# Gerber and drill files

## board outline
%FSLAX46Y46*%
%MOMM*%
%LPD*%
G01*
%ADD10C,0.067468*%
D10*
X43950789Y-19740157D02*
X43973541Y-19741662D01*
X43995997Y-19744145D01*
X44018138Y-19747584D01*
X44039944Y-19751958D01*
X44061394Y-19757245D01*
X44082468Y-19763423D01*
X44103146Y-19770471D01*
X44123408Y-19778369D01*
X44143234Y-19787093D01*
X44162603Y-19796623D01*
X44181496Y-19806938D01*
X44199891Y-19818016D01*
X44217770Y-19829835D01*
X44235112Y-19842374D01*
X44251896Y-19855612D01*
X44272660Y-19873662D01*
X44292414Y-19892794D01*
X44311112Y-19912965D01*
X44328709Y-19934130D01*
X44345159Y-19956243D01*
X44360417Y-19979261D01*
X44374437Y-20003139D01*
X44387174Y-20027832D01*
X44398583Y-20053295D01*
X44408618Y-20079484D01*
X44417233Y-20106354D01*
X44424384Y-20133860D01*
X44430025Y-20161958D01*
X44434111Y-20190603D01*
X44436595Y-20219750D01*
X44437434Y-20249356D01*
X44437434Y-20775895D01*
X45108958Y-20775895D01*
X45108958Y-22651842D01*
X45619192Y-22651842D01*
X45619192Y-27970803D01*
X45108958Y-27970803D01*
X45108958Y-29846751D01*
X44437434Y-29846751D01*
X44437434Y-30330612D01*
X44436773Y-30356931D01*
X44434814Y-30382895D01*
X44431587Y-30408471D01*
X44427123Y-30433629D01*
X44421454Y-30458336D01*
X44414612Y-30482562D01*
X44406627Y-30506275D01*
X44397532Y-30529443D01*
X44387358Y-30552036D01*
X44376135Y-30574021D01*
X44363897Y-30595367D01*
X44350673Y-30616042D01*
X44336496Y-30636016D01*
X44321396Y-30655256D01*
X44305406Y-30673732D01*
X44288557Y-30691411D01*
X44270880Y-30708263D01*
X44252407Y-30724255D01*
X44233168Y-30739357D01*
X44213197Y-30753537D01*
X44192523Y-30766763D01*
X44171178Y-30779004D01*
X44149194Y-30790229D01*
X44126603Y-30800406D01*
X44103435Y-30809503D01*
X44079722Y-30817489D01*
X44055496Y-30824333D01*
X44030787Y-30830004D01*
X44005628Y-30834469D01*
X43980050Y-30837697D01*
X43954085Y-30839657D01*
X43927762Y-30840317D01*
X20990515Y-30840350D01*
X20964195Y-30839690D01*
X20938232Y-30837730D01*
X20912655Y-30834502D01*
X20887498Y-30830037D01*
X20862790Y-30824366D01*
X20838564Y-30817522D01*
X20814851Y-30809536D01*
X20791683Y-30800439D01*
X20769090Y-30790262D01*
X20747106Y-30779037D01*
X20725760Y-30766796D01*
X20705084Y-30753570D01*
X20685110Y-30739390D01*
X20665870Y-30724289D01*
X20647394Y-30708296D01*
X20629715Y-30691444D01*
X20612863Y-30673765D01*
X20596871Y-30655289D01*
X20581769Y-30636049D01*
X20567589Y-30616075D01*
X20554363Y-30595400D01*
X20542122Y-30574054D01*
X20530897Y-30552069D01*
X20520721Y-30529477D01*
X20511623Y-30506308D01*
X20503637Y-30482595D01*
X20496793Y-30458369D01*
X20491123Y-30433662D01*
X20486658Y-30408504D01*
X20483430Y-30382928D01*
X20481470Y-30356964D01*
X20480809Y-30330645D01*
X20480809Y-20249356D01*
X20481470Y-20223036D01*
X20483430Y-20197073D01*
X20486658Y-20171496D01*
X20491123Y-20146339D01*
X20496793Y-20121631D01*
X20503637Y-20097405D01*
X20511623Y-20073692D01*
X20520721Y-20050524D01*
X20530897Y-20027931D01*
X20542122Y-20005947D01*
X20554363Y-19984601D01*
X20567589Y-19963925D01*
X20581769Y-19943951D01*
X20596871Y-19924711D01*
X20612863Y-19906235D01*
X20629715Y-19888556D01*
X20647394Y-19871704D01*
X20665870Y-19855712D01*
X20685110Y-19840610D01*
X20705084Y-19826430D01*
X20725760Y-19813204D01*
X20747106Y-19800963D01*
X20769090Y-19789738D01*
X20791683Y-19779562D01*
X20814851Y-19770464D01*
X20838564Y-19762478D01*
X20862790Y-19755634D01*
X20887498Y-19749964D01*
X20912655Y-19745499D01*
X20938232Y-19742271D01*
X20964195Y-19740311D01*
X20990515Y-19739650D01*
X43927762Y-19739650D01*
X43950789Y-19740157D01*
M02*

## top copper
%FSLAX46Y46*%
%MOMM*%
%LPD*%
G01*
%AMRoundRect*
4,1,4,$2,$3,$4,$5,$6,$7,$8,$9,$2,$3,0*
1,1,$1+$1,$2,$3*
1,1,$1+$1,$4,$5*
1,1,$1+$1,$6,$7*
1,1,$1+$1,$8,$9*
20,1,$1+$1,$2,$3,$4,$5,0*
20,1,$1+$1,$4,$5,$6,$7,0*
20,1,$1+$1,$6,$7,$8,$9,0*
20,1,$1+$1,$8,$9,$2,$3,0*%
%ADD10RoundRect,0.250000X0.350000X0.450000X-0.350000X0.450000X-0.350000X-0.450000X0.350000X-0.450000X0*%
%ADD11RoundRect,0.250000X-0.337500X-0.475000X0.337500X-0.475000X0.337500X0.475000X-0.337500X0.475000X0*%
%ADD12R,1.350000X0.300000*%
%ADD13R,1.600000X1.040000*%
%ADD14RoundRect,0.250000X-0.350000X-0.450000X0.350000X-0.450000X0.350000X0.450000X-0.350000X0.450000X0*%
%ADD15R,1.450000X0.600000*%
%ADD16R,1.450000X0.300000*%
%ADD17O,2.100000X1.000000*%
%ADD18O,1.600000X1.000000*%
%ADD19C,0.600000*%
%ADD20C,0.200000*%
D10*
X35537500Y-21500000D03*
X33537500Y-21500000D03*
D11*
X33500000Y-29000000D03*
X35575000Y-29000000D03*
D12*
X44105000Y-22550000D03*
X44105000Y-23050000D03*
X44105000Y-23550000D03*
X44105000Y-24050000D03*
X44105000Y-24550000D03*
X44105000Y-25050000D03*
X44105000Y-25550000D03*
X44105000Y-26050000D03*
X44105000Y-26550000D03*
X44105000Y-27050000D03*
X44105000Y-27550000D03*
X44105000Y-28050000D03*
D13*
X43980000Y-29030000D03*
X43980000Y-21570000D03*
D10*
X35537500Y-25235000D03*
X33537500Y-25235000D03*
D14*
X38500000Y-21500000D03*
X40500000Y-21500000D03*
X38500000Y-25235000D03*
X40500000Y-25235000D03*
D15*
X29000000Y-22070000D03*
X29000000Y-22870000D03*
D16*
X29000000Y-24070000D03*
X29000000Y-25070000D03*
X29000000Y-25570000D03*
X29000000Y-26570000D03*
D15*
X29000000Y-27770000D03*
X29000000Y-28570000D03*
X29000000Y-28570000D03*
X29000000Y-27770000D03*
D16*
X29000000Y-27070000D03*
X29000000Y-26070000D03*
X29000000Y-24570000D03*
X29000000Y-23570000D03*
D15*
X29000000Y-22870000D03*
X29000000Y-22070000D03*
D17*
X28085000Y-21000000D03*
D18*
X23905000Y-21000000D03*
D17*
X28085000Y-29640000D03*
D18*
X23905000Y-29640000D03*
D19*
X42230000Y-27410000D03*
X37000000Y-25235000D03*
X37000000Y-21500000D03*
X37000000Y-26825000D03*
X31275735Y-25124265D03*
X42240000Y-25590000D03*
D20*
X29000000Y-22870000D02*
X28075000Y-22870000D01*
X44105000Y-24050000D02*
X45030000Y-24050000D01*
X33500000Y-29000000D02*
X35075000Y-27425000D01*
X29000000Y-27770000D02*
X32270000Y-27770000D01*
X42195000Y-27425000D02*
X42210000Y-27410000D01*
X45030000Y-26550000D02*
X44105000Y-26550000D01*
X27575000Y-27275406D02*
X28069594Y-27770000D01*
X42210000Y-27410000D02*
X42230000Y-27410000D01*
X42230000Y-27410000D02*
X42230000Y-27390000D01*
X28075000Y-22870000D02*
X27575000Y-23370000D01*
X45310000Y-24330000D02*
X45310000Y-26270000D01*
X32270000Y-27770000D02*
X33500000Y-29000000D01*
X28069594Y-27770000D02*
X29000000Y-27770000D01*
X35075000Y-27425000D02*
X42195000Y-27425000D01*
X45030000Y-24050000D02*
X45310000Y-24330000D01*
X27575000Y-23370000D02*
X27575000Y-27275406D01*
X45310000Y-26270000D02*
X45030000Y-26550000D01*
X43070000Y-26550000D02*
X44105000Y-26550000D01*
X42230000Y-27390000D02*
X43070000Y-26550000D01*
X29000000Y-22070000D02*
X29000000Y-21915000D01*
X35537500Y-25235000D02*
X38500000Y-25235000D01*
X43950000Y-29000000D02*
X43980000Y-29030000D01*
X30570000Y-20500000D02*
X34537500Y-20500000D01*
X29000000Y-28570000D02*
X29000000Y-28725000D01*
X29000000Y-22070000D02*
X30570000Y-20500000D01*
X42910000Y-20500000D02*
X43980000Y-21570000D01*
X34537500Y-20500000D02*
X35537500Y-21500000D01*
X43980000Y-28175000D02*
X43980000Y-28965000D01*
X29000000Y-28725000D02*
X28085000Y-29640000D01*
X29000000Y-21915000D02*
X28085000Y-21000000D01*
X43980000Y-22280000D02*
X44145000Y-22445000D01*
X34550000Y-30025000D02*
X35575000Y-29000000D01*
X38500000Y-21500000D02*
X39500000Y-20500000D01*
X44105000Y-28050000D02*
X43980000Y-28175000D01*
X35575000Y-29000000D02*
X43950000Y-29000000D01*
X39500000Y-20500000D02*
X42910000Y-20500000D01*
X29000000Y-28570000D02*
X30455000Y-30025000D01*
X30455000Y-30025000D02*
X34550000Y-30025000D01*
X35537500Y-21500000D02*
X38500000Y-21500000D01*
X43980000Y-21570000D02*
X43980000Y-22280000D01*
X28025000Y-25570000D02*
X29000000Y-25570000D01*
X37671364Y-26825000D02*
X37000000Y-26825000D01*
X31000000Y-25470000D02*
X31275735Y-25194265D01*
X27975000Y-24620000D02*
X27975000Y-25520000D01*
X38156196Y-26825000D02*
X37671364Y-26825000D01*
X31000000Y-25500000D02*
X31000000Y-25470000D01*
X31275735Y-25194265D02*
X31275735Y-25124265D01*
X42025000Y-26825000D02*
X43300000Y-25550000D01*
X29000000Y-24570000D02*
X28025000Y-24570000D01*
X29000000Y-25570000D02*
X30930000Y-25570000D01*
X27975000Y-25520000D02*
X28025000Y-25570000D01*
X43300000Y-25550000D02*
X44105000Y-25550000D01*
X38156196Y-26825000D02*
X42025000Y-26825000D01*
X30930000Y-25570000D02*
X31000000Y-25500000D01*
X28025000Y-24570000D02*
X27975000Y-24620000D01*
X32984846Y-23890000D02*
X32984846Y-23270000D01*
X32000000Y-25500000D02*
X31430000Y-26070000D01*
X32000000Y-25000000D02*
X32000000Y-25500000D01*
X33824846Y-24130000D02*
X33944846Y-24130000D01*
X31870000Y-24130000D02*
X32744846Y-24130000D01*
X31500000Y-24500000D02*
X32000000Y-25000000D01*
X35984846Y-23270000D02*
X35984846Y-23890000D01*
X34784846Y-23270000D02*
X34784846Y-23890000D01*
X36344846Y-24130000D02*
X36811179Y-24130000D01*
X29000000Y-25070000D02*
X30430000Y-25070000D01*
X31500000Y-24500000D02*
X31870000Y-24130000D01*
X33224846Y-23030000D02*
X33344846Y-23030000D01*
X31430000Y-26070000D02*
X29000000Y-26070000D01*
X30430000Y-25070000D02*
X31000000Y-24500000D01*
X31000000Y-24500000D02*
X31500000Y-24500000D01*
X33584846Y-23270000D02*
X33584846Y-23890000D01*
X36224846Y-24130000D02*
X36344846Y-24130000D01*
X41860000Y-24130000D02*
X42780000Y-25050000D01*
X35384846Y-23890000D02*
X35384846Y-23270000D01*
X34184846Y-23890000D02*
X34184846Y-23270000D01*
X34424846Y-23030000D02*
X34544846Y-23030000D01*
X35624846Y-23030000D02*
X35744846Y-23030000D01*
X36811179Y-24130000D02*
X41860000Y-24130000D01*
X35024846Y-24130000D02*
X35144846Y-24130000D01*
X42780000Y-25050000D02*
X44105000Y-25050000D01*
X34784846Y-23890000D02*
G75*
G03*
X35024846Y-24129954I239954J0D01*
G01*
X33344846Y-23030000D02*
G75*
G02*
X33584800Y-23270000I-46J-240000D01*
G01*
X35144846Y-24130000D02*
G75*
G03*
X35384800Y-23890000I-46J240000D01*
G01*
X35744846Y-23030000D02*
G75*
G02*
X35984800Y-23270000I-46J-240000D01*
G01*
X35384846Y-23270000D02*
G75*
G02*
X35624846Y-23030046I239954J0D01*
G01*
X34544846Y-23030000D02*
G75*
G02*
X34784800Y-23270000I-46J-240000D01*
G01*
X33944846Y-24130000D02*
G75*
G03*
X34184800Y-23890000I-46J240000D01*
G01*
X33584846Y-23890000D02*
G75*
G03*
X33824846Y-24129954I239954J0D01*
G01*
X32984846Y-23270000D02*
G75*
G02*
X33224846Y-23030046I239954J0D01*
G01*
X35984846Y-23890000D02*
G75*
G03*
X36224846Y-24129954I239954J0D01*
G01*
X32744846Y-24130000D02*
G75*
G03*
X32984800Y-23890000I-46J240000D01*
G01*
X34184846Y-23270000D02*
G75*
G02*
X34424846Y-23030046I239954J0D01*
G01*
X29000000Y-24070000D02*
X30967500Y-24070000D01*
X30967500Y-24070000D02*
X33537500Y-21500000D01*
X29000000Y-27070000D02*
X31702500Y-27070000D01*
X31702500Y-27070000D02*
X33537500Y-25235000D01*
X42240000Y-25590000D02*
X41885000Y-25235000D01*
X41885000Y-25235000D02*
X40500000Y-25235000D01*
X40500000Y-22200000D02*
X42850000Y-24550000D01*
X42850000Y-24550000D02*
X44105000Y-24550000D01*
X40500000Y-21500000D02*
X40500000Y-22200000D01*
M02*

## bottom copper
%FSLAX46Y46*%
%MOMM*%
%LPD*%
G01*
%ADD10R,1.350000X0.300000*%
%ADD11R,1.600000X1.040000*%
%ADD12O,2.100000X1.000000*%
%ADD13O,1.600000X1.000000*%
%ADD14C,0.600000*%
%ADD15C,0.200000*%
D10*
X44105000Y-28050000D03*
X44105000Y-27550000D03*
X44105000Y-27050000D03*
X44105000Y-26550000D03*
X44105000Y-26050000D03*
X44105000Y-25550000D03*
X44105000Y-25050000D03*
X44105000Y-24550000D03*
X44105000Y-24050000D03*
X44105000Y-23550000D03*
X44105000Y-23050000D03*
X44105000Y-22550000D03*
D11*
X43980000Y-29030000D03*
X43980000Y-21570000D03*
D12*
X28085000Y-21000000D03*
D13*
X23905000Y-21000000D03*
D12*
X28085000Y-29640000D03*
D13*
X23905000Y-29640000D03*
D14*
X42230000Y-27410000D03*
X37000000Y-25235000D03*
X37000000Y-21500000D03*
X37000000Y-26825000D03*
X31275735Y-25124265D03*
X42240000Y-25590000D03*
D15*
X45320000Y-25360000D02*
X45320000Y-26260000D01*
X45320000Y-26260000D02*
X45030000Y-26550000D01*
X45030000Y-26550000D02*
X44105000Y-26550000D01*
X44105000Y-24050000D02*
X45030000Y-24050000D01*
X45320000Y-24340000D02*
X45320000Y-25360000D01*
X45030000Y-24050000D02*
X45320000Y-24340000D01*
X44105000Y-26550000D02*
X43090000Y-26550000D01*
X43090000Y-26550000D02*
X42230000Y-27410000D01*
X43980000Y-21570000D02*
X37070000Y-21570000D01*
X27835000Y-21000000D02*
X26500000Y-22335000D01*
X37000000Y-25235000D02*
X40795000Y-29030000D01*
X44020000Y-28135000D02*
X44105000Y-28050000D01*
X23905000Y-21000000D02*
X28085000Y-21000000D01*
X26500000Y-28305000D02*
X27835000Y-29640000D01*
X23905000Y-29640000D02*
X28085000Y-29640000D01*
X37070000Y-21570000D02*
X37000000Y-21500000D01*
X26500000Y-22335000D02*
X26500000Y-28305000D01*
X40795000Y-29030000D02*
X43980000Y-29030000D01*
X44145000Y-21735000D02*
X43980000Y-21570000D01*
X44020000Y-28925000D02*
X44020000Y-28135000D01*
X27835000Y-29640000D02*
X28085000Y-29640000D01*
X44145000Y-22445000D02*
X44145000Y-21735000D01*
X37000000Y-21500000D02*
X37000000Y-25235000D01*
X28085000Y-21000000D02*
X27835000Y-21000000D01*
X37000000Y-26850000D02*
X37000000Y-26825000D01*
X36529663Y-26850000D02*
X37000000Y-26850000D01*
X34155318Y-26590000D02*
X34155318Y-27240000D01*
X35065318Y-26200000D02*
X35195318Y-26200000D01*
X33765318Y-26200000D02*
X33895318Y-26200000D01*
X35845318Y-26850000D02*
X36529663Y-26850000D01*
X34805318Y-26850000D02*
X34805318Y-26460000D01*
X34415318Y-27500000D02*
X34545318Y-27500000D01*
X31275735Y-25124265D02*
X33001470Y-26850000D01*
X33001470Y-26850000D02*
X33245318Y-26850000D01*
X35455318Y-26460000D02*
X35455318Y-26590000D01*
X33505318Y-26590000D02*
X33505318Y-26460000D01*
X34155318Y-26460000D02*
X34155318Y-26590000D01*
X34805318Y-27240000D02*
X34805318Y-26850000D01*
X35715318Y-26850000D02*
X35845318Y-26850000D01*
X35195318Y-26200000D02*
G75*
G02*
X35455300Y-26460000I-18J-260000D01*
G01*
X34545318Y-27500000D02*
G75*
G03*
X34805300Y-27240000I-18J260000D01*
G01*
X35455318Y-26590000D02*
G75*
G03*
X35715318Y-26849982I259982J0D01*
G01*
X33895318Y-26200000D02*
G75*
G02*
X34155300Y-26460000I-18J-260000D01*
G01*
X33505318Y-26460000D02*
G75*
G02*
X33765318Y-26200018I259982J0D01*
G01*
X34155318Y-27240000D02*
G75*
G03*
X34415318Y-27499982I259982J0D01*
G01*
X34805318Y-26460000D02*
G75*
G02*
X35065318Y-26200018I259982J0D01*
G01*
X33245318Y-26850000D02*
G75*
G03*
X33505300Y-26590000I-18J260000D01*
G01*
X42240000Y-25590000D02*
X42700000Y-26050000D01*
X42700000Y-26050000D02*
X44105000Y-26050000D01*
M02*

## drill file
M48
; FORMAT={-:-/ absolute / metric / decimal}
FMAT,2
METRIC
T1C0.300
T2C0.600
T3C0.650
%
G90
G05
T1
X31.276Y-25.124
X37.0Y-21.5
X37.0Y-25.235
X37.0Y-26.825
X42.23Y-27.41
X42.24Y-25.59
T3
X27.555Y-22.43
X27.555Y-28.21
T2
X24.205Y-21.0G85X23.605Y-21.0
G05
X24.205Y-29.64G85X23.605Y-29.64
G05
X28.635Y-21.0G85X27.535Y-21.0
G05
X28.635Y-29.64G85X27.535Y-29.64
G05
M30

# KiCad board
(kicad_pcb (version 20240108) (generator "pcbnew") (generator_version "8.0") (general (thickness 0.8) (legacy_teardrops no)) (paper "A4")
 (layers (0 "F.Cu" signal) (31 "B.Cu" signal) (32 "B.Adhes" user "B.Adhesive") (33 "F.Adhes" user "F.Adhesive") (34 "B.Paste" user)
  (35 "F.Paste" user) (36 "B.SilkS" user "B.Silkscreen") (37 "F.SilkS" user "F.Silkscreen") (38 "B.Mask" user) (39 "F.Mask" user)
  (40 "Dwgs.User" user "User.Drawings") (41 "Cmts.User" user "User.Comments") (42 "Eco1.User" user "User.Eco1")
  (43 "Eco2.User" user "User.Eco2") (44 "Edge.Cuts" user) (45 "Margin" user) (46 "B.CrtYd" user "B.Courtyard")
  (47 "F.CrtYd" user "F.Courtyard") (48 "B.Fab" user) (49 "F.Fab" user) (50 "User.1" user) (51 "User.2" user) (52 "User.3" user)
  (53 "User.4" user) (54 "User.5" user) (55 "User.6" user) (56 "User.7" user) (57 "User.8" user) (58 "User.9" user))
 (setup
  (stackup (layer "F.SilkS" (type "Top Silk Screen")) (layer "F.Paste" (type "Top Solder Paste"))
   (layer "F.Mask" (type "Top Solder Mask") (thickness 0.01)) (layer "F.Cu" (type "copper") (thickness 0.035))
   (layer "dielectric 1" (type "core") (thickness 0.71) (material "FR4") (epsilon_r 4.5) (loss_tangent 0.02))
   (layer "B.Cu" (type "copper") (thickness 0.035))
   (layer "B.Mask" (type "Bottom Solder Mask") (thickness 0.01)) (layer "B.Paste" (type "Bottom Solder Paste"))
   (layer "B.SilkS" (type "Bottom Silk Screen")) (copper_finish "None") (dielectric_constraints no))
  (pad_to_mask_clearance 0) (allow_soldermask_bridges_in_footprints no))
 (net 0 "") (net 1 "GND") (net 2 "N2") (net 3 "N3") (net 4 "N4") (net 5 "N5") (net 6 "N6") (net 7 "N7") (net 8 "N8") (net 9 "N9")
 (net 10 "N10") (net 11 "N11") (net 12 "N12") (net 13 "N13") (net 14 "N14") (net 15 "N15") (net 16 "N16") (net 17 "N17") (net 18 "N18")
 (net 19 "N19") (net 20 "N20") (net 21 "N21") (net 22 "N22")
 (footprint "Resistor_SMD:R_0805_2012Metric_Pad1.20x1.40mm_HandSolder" (layer "F.Cu") (at 34.5375 21.5 180)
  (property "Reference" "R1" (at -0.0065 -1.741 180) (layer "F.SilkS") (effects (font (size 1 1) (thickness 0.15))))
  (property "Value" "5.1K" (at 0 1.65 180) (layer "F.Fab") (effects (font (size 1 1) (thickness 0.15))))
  (pad "1" smd roundrect (at -1 0 180) (size 1.2 1.4) (layers "F.Cu" "F.Paste" "F.Mask") (roundrect_rratio 0.208333) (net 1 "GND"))
  (pad "2" smd roundrect (at 1 0 180) (size 1.2 1.4) (layers "F.Cu" "F.Paste" "F.Mask") (roundrect_rratio 0.208333) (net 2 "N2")))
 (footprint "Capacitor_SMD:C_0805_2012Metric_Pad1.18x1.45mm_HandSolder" (layer "F.Cu") (at 34.5375 29)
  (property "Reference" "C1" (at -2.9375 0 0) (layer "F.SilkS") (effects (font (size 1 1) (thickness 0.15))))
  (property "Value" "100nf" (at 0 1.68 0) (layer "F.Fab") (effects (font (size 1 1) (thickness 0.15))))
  (pad "1" smd roundrect (at -1.0375 0) (size 1.175 1.45) (layers "F.Cu" "F.Paste" "F.Mask") (roundrect_rratio 0.212766) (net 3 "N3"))
  (pad "2" smd roundrect (at 1.0375 0) (size 1.175 1.45) (layers "F.Cu" "F.Paste" "F.Mask") (roundrect_rratio 0.212766) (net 1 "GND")))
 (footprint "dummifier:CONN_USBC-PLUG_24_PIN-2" (layer "F.Cu") (at 44.95 25.33 90)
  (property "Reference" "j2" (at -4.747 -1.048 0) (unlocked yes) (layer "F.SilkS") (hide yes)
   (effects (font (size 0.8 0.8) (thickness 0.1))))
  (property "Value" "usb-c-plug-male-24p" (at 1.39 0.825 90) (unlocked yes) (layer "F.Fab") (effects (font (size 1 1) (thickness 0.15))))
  (pad "A1" smd rect (at 2.78 -0.845 90) (size 0.3 1.35) (layers "F.Cu" "F.Paste" "F.Mask") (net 1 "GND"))
  (pad "A2" smd rect (at 2.28 -0.845 90) (size 0.3 1.35) (layers "F.Cu" "F.Paste" "F.Mask") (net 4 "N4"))
  (pad "A3" smd rect (at 1.78 -0.845 90) (size 0.3 1.35) (layers "F.Cu" "F.Paste" "F.Mask") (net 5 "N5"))
  (pad "A4" smd rect (at 1.28 -0.845 90) (size 0.3 1.35) (layers "F.Cu" "F.Paste" "F.Mask") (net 3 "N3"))
  (pad "A5" smd rect (at 0.78 -0.845 90) (size 0.3 1.35) (layers "F.Cu" "F.Paste" "F.Mask") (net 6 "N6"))
  (pad "A6" smd rect (at 0.28 -0.845 90) (size 0.3 1.35) (layers "F.Cu" "F.Paste" "F.Mask") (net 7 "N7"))
  (pad "A7" smd rect (at -0.22 -0.845 90) (size 0.3 1.35) (layers "F.Cu" "F.Paste" "F.Mask") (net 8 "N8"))
  (pad "A8" smd rect (at -0.72 -0.845 90) (size 0.3 1.35) (layers "F.Cu" "F.Paste" "F.Mask") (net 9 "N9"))
  (pad "A9" smd rect (at -1.22 -0.845 90) (size 0.3 1.35) (layers "F.Cu" "F.Paste" "F.Mask") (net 3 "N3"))
  (pad "A10" smd rect (at -1.72 -0.845 90) (size 0.3 1.35) (layers "F.Cu" "F.Paste" "F.Mask") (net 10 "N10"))
  (pad "A11" smd rect (at -2.22 -0.845 90) (size 0.3 1.35) (layers "F.Cu" "F.Paste" "F.Mask") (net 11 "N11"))
  (pad "A12" smd rect (at -2.72 -0.845 90) (size 0.3 1.35) (layers "F.Cu" "F.Paste" "F.Mask") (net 1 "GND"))
  (pad "B1" smd rect (at -2.72 -0.845 90) (size 0.3 1.35) (layers "B.Cu" "B.Paste" "B.Mask") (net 1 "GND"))
  (pad "B2" smd rect (at -2.22 -0.845 90) (size 0.3 1.35) (layers "B.Cu" "B.Paste" "B.Mask") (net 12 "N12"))
  (pad "B3" smd rect (at -1.72 -0.845 90) (size 0.3 1.35) (layers "B.Cu" "B.Paste" "B.Mask") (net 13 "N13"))
  (pad "B4" smd rect (at -1.22 -0.845 90) (size 0.3 1.35) (layers "B.Cu" "B.Paste" "B.Mask") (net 3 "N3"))
  (pad "B5" smd rect (at -0.72 -0.845 90) (size 0.3 1.35) (layers "B.Cu" "B.Paste" "B.Mask") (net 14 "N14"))
  (pad "B6" smd rect (at -0.22 -0.845 90) (size 0.3 1.35) (layers "B.Cu" "B.Paste" "B.Mask") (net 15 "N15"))
  (pad "B7" smd rect (at 0.28 -0.845 90) (size 0.3 1.35) (layers "B.Cu" "B.Paste" "B.Mask") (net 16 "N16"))
  (pad "B8" smd rect (at 0.78 -0.845 90) (size 0.3 1.35) (layers "B.Cu" "B.Paste" "B.Mask") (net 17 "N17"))
  (pad "B9" smd rect (at 1.28 -0.845 90) (size 0.3 1.35) (layers "B.Cu" "B.Paste" "B.Mask") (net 3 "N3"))
  (pad "B10" smd rect (at 1.78 -0.845 90) (size 0.3 1.35) (layers "B.Cu" "B.Paste" "B.Mask") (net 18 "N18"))
  (pad "B11" smd rect (at 2.28 -0.845 90) (size 0.3 1.35) (layers "B.Cu" "B.Paste" "B.Mask") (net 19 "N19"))
  (pad "B12" smd rect (at 2.78 -0.845 90) (size 0.3 1.35) (layers "B.Cu" "B.Paste" "B.Mask") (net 1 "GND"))
  (pad "S" smd rect (at -3.7 -0.97 90) (size 1.04 1.6) (layers "F.Cu" "F.Paste" "F.Mask") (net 1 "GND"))
  (pad "S" smd rect (at -3.7 -0.97 90) (size 1.04 1.6) (layers "B.Cu" "B.Paste" "B.Mask") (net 1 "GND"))
  (pad "S" smd rect (at 3.76 -0.97 90) (size 1.04 1.6) (layers "F.Cu" "F.Paste" "F.Mask") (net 1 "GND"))
  (pad "S" smd rect (at 3.76 -0.97 90) (size 1.04 1.6) (layers "B.Cu" "B.Paste" "B.Mask") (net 1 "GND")))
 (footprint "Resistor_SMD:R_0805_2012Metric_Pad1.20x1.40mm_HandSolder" (layer "F.Cu") (at 34.5375 25.235 180)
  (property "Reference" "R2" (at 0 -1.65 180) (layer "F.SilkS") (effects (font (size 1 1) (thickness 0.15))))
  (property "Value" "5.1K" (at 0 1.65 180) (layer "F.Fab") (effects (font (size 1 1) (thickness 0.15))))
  (pad "1" smd roundrect (at -1 0 180) (size 1.2 1.4) (layers "F.Cu" "F.Paste" "F.Mask") (roundrect_rratio 0.208333) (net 1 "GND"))
  (pad "2" smd roundrect (at 1 0 180) (size 1.2 1.4) (layers "F.Cu" "F.Paste" "F.Mask") (roundrect_rratio 0.208333) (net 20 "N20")))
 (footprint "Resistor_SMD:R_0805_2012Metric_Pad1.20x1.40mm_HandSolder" (layer "F.Cu") (at 39.5 21.5)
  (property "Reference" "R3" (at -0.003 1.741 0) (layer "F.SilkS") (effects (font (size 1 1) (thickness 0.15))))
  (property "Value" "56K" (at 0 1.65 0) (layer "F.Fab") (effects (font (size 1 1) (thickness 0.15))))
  (pad "1" smd roundrect (at -1 0) (size 1.2 1.4) (layers "F.Cu" "F.Paste" "F.Mask") (roundrect_rratio 0.208333) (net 1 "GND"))
  (pad "2" smd roundrect (at 1 0) (size 1.2 1.4) (layers "F.Cu" "F.Paste" "F.Mask") (roundrect_rratio 0.208333) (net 6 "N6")))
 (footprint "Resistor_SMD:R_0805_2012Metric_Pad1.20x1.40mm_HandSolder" (layer "F.Cu") (at 39.5 25.235)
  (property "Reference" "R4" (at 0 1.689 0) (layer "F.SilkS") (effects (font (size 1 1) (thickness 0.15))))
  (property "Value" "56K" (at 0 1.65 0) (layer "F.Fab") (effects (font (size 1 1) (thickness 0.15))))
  (pad "1" smd roundrect (at -1 0) (size 1.2 1.4) (layers "F.Cu" "F.Paste" "F.Mask") (roundrect_rratio 0.208333) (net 1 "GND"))
  (pad "2" smd roundrect (at 1 0) (size 1.2 1.4) (layers "F.Cu" "F.Paste" "F.Mask") (roundrect_rratio 0.208333) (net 14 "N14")))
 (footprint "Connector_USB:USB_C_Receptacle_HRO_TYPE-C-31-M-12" (layer "F.Cu") (at 24.955 25.32 -90)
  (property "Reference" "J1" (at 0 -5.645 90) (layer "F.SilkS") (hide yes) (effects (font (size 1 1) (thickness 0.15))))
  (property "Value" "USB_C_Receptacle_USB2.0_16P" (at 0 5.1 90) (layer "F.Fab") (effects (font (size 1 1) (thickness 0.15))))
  (pad "" np_thru_hole circle (at -2.89 -2.6 270) (size 0.65 0.65) (drill 0.65) (layers "*.Cu" "*.Mask"))
  (pad "" np_thru_hole circle (at 2.89 -2.6 270) (size 0.65 0.65) (drill 0.65) (layers "*.Cu" "*.Mask"))
  (pad "A1" smd rect (at -3.25 -4.045 270) (size 0.6 1.45) (layers "F.Cu" "F.Paste" "F.Mask") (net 1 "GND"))
  (pad "A4" smd rect (at -2.45 -4.045 270) (size 0.6 1.45) (layers "F.Cu" "F.Paste" "F.Mask") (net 3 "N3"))
  (pad "A5" smd rect (at -1.25 -4.045 270) (size 0.3 1.45) (layers "F.Cu" "F.Paste" "F.Mask") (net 2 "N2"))
  (pad "A6" smd rect (at -0.25 -4.045 270) (size 0.3 1.45) (layers "F.Cu" "F.Paste" "F.Mask") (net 7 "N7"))
  (pad "A7" smd rect (at 0.25 -4.045 270) (size 0.3 1.45) (layers "F.Cu" "F.Paste" "F.Mask") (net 8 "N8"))
  (pad "A8" smd rect (at 1.25 -4.045 270) (size 0.3 1.45) (layers "F.Cu" "F.Paste" "F.Mask") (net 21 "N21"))
  (pad "A9" smd rect (at 2.45 -4.045 270) (size 0.6 1.45) (layers "F.Cu" "F.Paste" "F.Mask") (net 3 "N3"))
  (pad "A12" smd rect (at 3.25 -4.045 270) (size 0.6 1.45) (layers "F.Cu" "F.Paste" "F.Mask") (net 1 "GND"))
  (pad "B1" smd rect (at 3.25 -4.045 270) (size 0.6 1.45) (layers "F.Cu" "F.Paste" "F.Mask") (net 1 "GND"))
  (pad "B4" smd rect (at 2.45 -4.045 270) (size 0.6 1.45) (layers "F.Cu" "F.Paste" "F.Mask") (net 3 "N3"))
  (pad "B5" smd rect (at 1.75 -4.045 270) (size 0.3 1.45) (layers "F.Cu" "F.Paste" "F.Mask") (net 20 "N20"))
  (pad "B6" smd rect (at 0.75 -4.045 270) (size 0.3 1.45) (layers "F.Cu" "F.Paste" "F.Mask") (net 7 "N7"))
  (pad "B7" smd rect (at -0.75 -4.045 270) (size 0.3 1.45) (layers "F.Cu" "F.Paste" "F.Mask") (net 8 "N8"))
  (pad "B8" smd rect (at -1.75 -4.045 270) (size 0.3 1.45) (layers "F.Cu" "F.Paste" "F.Mask") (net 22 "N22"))
  (pad "B9" smd rect (at -2.45 -4.045 270) (size 0.6 1.45) (layers "F.Cu" "F.Paste" "F.Mask") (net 3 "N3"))
  (pad "B12" smd rect (at -3.25 -4.045 270) (size 0.6 1.45) (layers "F.Cu" "F.Paste" "F.Mask") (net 1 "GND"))
  (pad "S1" thru_hole oval (at -4.32 -3.13 270) (size 1 2.1) (drill oval 0.6 1.7) (layers "*.Cu" "*.Mask") (remove_unused_layers no)
   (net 1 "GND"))
  (pad "S1" thru_hole oval (at -4.32 1.05 270) (size 1 1.6) (drill oval 0.6 1.2) (layers "*.Cu" "*.Mask") (remove_unused_layers no)
   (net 1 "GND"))
  (pad "S1" thru_hole oval (at 4.32 -3.13 270) (size 1 2.1) (drill oval 0.6 1.7) (layers "*.Cu" "*.Mask") (remove_unused_layers no)
   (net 1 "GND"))
  (pad "S1" thru_hole oval (at 4.32 1.05 270) (size 1 1.6) (drill oval 0.6 1.2) (layers "*.Cu" "*.Mask") (remove_unused_layers no)
   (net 1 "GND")))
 (gr_poly
  (pts (xy 43.950789 19.740157) (xy 43.973541 19.741662) (xy 43.995997 19.744145) (xy 44.018138 19.747584) (xy 44.039944 19.751958)
   (xy 44.061394 19.757245) (xy 44.082468 19.763423) (xy 44.103146 19.770471) (xy 44.123408 19.778369) (xy 44.143234 19.787093)
   (xy 44.162603 19.796623) (xy 44.181496 19.806938) (xy 44.199891 19.818016) (xy 44.21777 19.829835) (xy 44.235112 19.842374)
   (xy 44.251896 19.855612) (xy 44.27266 19.873662) (xy 44.292414 19.892794) (xy 44.311112 19.912965) (xy 44.328709 19.93413)
   (xy 44.345159 19.956243) (xy 44.360417 19.979261) (xy 44.374437 20.003139) (xy 44.387174 20.027832) (xy 44.398583 20.053295)
   (xy 44.408618 20.079484) (xy 44.417233 20.106354) (xy 44.424384 20.13386) (xy 44.430025 20.161958) (xy 44.434111 20.190603)
   (xy 44.436595 20.21975) (xy 44.437434 20.249356) (xy 44.437434 20.775895) (xy 45.108958 20.775895) (xy 45.108958 22.651842)
   (xy 45.619192 22.651842) (xy 45.619192 27.970803) (xy 45.108958 27.970803) (xy 45.108958 29.846751) (xy 44.437434 29.846751)
   (xy 44.437434 30.330612) (xy 44.436773 30.356931) (xy 44.434814 30.382895) (xy 44.431587 30.408471) (xy 44.427123 30.433629)
   (xy 44.421454 30.458336) (xy 44.414612 30.482562) (xy 44.406627 30.506275) (xy 44.397532 30.529443) (xy 44.387358 30.552036)
   (xy 44.376135 30.574021) (xy 44.363897 30.595367) (xy 44.350673 30.616042) (xy 44.336496 30.636016) (xy 44.321396 30.655256)
   (xy 44.305406 30.673732) (xy 44.288557 30.691411) (xy 44.27088 30.708263) (xy 44.252407 30.724255) (xy 44.233168 30.739357)
   (xy 44.213197 30.753537) (xy 44.192523 30.766763) (xy 44.171178 30.779004) (xy 44.149194 30.790229) (xy 44.126603 30.800406)
   (xy 44.103435 30.809503) (xy 44.079722 30.817489) (xy 44.055496 30.824333) (xy 44.030787 30.830004) (xy 44.005628 30.834469)
   (xy 43.98005 30.837697) (xy 43.954085 30.839657) (xy 43.927762 30.840317) (xy 20.990515 30.84035) (xy 20.964195 30.83969)
   (xy 20.938232 30.83773) (xy 20.912655 30.834502) (xy 20.887498 30.830037) (xy 20.86279 30.824366) (xy 20.838564 30.817522)
   (xy 20.814851 30.809536) (xy 20.791683 30.800439) (xy 20.76909 30.790262) (xy 20.747106 30.779037) (xy 20.72576 30.766796)
   (xy 20.705084 30.75357) (xy 20.68511 30.73939) (xy 20.66587 30.724289) (xy 20.647394 30.708296) (xy 20.629715 30.691444)
   (xy 20.612863 30.673765) (xy 20.596871 30.655289) (xy 20.581769 30.636049) (xy 20.567589 30.616075) (xy 20.554363 30.5954)
   (xy 20.542122 30.574054) (xy 20.530897 30.552069) (xy 20.520721 30.529477) (xy 20.511623 30.506308) (xy 20.503637 30.482595)
   (xy 20.496793 30.458369) (xy 20.491123 30.433662) (xy 20.486658 30.408504) (xy 20.48343 30.382928) (xy 20.48147 30.356964)
   (xy 20.480809 30.330645) (xy 20.480809 20.249356) (xy 20.48147 20.223036) (xy 20.48343 20.197073) (xy 20.486658 20.171496)
   (xy 20.491123 20.146339) (xy 20.496793 20.121631) (xy 20.503637 20.097405) (xy 20.511623 20.073692) (xy 20.520721 20.050524)
   (xy 20.530897 20.027931) (xy 20.542122 20.005947) (xy 20.554363 19.984601) (xy 20.567589 19.963925) (xy 20.581769 19.943951)
   (xy 20.596871 19.924711) (xy 20.612863 19.906235) (xy 20.629715 19.888556) (xy 20.647394 19.871704) (xy 20.66587 19.855712)
   (xy 20.68511 19.84061) (xy 20.705084 19.82643) (xy 20.72576 19.813204) (xy 20.747106 19.800963) (xy 20.76909 19.789738)
   (xy 20.791683 19.779562) (xy 20.814851 19.770464) (xy 20.838564 19.762478) (xy 20.86279 19.755634) (xy 20.887498 19.749964)
   (xy 20.912655 19.745499) (xy 20.938232 19.742271) (xy 20.964195 19.740311) (xy 20.990515 19.73965) (xy 43.927762 19.73965))
  (stroke (width 0.067468) (type solid) (color 255 0 0 1)) (fill none) (layer "Edge.Cuts"))
 (segment (start 29 22.87) (end 28.075 22.87) (width 0.2) (layer "F.Cu") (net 3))
 (segment (start 44.105 24.05) (end 45.03 24.05) (width 0.2) (layer "F.Cu") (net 3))
 (segment (start 33.5 29) (end 35.075 27.425) (width 0.2) (layer "F.Cu") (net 3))
 (segment (start 29 27.77) (end 32.27 27.77) (width 0.2) (layer "F.Cu") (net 3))
 (segment (start 42.195 27.425) (end 42.21 27.41) (width 0.2) (layer "F.Cu") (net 3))
 (segment (start 45.03 26.55) (end 44.105 26.55) (width 0.2) (layer "F.Cu") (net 3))
 (segment (start 27.575 27.275406) (end 28.069594 27.77) (width 0.2) (layer "F.Cu") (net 3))
 (segment (start 42.21 27.41) (end 42.23 27.41) (width 0.2) (layer "F.Cu") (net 3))
 (segment (start 42.23 27.41) (end 42.23 27.39) (width 0.2) (layer "F.Cu") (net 3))
 (segment (start 28.075 22.87) (end 27.575 23.37) (width 0.2) (layer "F.Cu") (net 3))
 (segment (start 45.31 24.33) (end 45.31 26.27) (width 0.2) (layer "F.Cu") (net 3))
 (segment (start 32.27 27.77) (end 33.5 29) (width 0.2) (layer "F.Cu") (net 3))
 (segment (start 28.069594 27.77) (end 29 27.77) (width 0.2) (layer "F.Cu") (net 3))
 (segment (start 35.075 27.425) (end 42.195 27.425) (width 0.2) (layer "F.Cu") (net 3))
 (segment (start 45.03 24.05) (end 45.31 24.33) (width 0.2) (layer "F.Cu") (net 3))
 (segment (start 27.575 23.37) (end 27.575 27.275406) (width 0.2) (layer "F.Cu") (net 3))
 (segment (start 45.31 26.27) (end 45.03 26.55) (width 0.2) (layer "F.Cu") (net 3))
 (segment (start 43.07 26.55) (end 44.105 26.55) (width 0.2) (layer "F.Cu") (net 3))
 (segment (start 42.23 27.39) (end 43.07 26.55) (width 0.2) (layer "F.Cu") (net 3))
 (via (at 42.23 27.41) (size 0.6) (drill 0.3) (layers "F.Cu" "B.Cu") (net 3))
 (segment (start 45.32 25.36) (end 45.32 26.26) (width 0.2) (layer "B.Cu") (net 3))
 (segment (start 45.32 26.26) (end 45.03 26.55) (width 0.2) (layer "B.Cu") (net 3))
 (segment (start 45.03 26.55) (end 44.105 26.55) (width 0.2) (layer "B.Cu") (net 3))
 (segment (start 44.105 24.05) (end 45.03 24.05) (width 0.2) (layer "B.Cu") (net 3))
 (segment (start 45.32 24.34) (end 45.32 25.36) (width 0.2) (layer "B.Cu") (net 3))
 (segment (start 45.03 24.05) (end 45.32 24.34) (width 0.2) (layer "B.Cu") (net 3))
 (segment (start 44.105 26.55) (end 43.09 26.55) (width 0.2) (layer "B.Cu") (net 3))
 (segment (start 43.09 26.55) (end 42.23 27.41) (width 0.2) (layer "B.Cu") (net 3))
 (segment (start 29 22.07) (end 29 21.915) (width 0.2) (layer "F.Cu") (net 1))
 (segment (start 35.5375 25.235) (end 38.5 25.235) (width 0.2) (layer "F.Cu") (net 1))
 (segment (start 43.95 29) (end 43.98 29.03) (width 0.2) (layer "F.Cu") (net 1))
 (segment (start 30.57 20.5) (end 34.5375 20.5) (width 0.2) (layer "F.Cu") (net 1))
 (segment (start 29 28.57) (end 29 28.725) (width 0.2) (layer "F.Cu") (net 1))
 (segment (start 29 22.07) (end 30.57 20.5) (width 0.2) (layer "F.Cu") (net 1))
 (segment (start 42.91 20.5) (end 43.98 21.57) (width 0.2) (layer "F.Cu") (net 1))
 (segment (start 34.5375 20.5) (end 35.5375 21.5) (width 0.2) (layer "F.Cu") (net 1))
 (segment (start 43.98 28.175) (end 43.98 28.965) (width 0.2) (layer "F.Cu") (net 1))
 (segment (start 29 28.725) (end 28.085 29.64) (width 0.2) (layer "F.Cu") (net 1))
 (segment (start 29 21.915) (end 28.085 21) (width 0.2) (layer "F.Cu") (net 1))
 (segment (start 43.98 22.28) (end 44.145 22.445) (width 0.2) (layer "F.Cu") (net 1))
 (segment (start 34.55 30.025) (end 35.575 29) (width 0.2) (layer "F.Cu") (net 1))
 (segment (start 38.5 21.5) (end 39.5 20.5) (width 0.2) (layer "F.Cu") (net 1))
 (segment (start 44.105 28.05) (end 43.98 28.175) (width 0.2) (layer "F.Cu") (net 1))
 (segment (start 35.575 29) (end 43.95 29) (width 0.2) (layer "F.Cu") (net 1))
 (segment (start 39.5 20.5) (end 42.91 20.5) (width 0.2) (layer "F.Cu") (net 1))
 (segment (start 29 28.57) (end 30.455 30.025) (width 0.2) (layer "F.Cu") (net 1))
 (segment (start 30.455 30.025) (end 34.55 30.025) (width 0.2) (layer "F.Cu") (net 1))
 (segment (start 35.5375 21.5) (end 38.5 21.5) (width 0.2) (layer "F.Cu") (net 1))
 (segment (start 43.98 21.57) (end 43.98 22.28) (width 0.2) (layer "F.Cu") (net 1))
 (via (at 37 25.235) (size 0.6) (drill 0.3) (layers "F.Cu" "B.Cu") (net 1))
 (via (at 37 21.5) (size 0.6) (drill 0.3) (layers "F.Cu" "B.Cu") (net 1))
 (segment (start 43.98 21.57) (end 37.07 21.57) (width 0.2) (layer "B.Cu") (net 1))
 (segment (start 27.835 21) (end 26.5 22.335) (width 0.2) (layer "B.Cu") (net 1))
 (segment (start 37 25.235) (end 40.795 29.03) (width 0.2) (layer "B.Cu") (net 1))
 (segment (start 44.02 28.135) (end 44.105 28.05) (width 0.2) (layer "B.Cu") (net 1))
 (segment (start 23.905 21) (end 28.085 21) (width 0.2) (layer "B.Cu") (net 1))
 (segment (start 26.5 28.305) (end 27.835 29.64) (width 0.2) (layer "B.Cu") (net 1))
 (segment (start 23.905 29.64) (end 28.085 29.64) (width 0.2) (layer "B.Cu") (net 1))
 (segment (start 37.07 21.57) (end 37 21.5) (width 0.2) (layer "B.Cu") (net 1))
 (segment (start 26.5 22.335) (end 26.5 28.305) (width 0.2) (layer "B.Cu") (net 1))
 (segment (start 40.795 29.03) (end 43.98 29.03) (width 0.2) (layer "B.Cu") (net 1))
 (segment (start 44.145 21.735) (end 43.98 21.57) (width 0.2) (layer "B.Cu") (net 1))
 (segment (start 44.02 28.925) (end 44.02 28.135) (width 0.2) (layer "B.Cu") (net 1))
 (segment (start 27.835 29.64) (end 28.085 29.64) (width 0.2) (layer "B.Cu") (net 1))
 (segment (start 44.145 22.445) (end 44.145 21.735) (width 0.2) (layer "B.Cu") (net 1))
 (segment (start 37 21.5) (end 37 25.235) (width 0.2) (layer "B.Cu") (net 1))
 (segment (start 28.085 21) (end 27.835 21) (width 0.2) (layer "B.Cu") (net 1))
 (segment (start 28.025 25.57) (end 29 25.57) (width 0.2) (layer "F.Cu") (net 8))
 (segment (start 37.671364 26.825) (end 37 26.825) (width 0.2) (layer "F.Cu") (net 8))
 (segment (start 31 25.47) (end 31.275735 25.194265) (width 0.2) (layer "F.Cu") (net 8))
 (segment (start 27.975 24.62) (end 27.975 25.52) (width 0.2) (layer "F.Cu") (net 8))
 (segment (start 38.156196 26.825) (end 37.671364 26.825) (width 0.2) (layer "F.Cu") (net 8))
 (segment (start 31 25.5) (end 31 25.47) (width 0.2) (layer "F.Cu") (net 8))
 (segment (start 31.275735 25.194265) (end 31.275735 25.124265) (width 0.2) (layer "F.Cu") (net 8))
 (segment (start 42.025 26.825) (end 43.3 25.55) (width 0.2) (layer "F.Cu") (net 8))
 (segment (start 29 24.57) (end 28.025 24.57) (width 0.2) (layer "F.Cu") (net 8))
 (segment (start 29 25.57) (end 30.93 25.57) (width 0.2) (layer "F.Cu") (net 8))
 (segment (start 27.975 25.52) (end 28.025 25.57) (width 0.2) (layer "F.Cu") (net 8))
 (segment (start 43.3 25.55) (end 44.105 25.55) (width 0.2) (layer "F.Cu") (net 8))
 (segment (start 38.156196 26.825) (end 42.025 26.825) (width 0.2) (layer "F.Cu") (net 8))
 (segment (start 30.93 25.57) (end 31 25.5) (width 0.2) (layer "F.Cu") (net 8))
 (segment (start 28.025 24.57) (end 27.975 24.62) (width 0.2) (layer "F.Cu") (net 8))
 (via (at 37 26.825) (size 0.6) (drill 0.3) (layers "F.Cu" "B.Cu") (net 8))
 (via (at 31.275735 25.124265) (size 0.6) (drill 0.3) (layers "F.Cu" "B.Cu") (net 8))
 (segment (start 37 26.85) (end 37 26.825) (width 0.2) (layer "B.Cu") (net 8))
 (segment (start 36.529663 26.85) (end 37 26.85) (width 0.2) (layer "B.Cu") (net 8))
 (segment (start 34.155318 26.59) (end 34.155318 27.24) (width 0.2) (layer "B.Cu") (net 8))
 (segment (start 35.065318 26.2) (end 35.195318 26.2) (width 0.2) (layer "B.Cu") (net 8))
 (segment (start 33.765318 26.2) (end 33.895318 26.2) (width 0.2) (layer "B.Cu") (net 8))
 (segment (start 35.845318 26.85) (end 36.529663 26.85) (width 0.2) (layer "B.Cu") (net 8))
 (segment (start 34.805318 26.85) (end 34.805318 26.46) (width 0.2) (layer "B.Cu") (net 8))
 (segment (start 34.415318 27.5) (end 34.545318 27.5) (width 0.2) (layer "B.Cu") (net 8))
 (segment (start 31.275735 25.124265) (end 33.00147 26.85) (width 0.2) (layer "B.Cu") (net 8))
 (segment (start 33.00147 26.85) (end 33.245318 26.85) (width 0.2) (layer "B.Cu") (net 8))
 (segment (start 35.455318 26.46) (end 35.455318 26.59) (width 0.2) (layer "B.Cu") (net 8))
 (segment (start 33.505318 26.59) (end 33.505318 26.46) (width 0.2) (layer "B.Cu") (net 8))
 (segment (start 34.155318 26.46) (end 34.155318 26.59) (width 0.2) (layer "B.Cu") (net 8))
 (segment (start 34.805318 27.24) (end 34.805318 26.85) (width 0.2) (layer "B.Cu") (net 8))
 (segment (start 35.715318 26.85) (end 35.845318 26.85) (width 0.2) (layer "B.Cu") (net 8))
 (arc (start 35.195318 26.2) (mid 35.379166 26.276152) (end 35.455318 26.46) (width 0.2) (layer "B.Cu") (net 8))
 (arc (start 34.545318 27.5) (mid 34.729166 27.423848) (end 34.805318 27.24) (width 0.2) (layer "B.Cu") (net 8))
 (arc (start 35.455318 26.59) (mid 35.53147 26.773848) (end 35.715318 26.85) (width 0.2) (layer "B.Cu") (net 8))
 (arc (start 33.895318 26.2) (mid 34.079166 26.276152) (end 34.155318 26.46) (width 0.2) (layer "B.Cu") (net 8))
 (arc (start 33.505318 26.46) (mid 33.58147 26.276152) (end 33.765318 26.2) (width 0.2) (layer "B.Cu") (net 8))
 (arc (start 34.155318 27.24) (mid 34.23147 27.423848) (end 34.415318 27.5) (width 0.2) (layer "B.Cu") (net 8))
 (arc (start 34.805318 26.46) (mid 34.88147 26.276152) (end 35.065318 26.2) (width 0.2) (layer "B.Cu") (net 8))
 (arc (start 33.245318 26.85) (mid 33.429166 26.773848) (end 33.505318 26.59) (width 0.2) (layer "B.Cu") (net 8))
 (segment (start 32.984846 23.89) (end 32.984846 23.27) (width 0.2) (layer "F.Cu") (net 7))
 (segment (start 32 25.5) (end 31.43 26.07) (width 0.2) (layer "F.Cu") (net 7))
 (segment (start 32 25) (end 32 25.5) (width 0.2) (layer "F.Cu") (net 7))
 (segment (start 33.824846 24.13) (end 33.944846 24.13) (width 0.2) (layer "F.Cu") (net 7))
 (segment (start 31.87 24.13) (end 32.744846 24.13) (width 0.2) (layer "F.Cu") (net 7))
 (segment (start 31.5 24.5) (end 32 25) (width 0.2) (layer "F.Cu") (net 7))
 (segment (start 35.984846 23.27) (end 35.984846 23.89) (width 0.2) (layer "F.Cu") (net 7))
 (segment (start 34.784846 23.27) (end 34.784846 23.89) (width 0.2) (layer "F.Cu") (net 7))
 (segment (start 36.344846 24.13) (end 36.811179 24.13) (width 0.2) (layer "F.Cu") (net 7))
 (segment (start 29 25.07) (end 30.43 25.07) (width 0.2) (layer "F.Cu") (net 7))
 (segment (start 31.5 24.5) (end 31.87 24.13) (width 0.2) (layer "F.Cu") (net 7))
 (segment (start 33.224846 23.03) (end 33.344846 23.03) (width 0.2) (layer "F.Cu") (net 7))
 (segment (start 31.43 26.07) (end 29 26.07) (width 0.2) (layer "F.Cu") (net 7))
 (segment (start 30.43 25.07) (end 31 24.5) (width 0.2) (layer "F.Cu") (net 7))
 (segment (start 31 24.5) (end 31.5 24.5) (width 0.2) (layer "F.Cu") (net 7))
 (segment (start 33.584846 23.27) (end 33.584846 23.89) (width 0.2) (layer "F.Cu") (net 7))
 (segment (start 36.224846 24.13) (end 36.344846 24.13) (width 0.2) (layer "F.Cu") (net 7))
 (segment (start 41.86 24.13) (end 42.78 25.05) (width 0.2) (layer "F.Cu") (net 7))
 (segment (start 35.384846 23.89) (end 35.384846 23.27) (width 0.2) (layer "F.Cu") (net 7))
 (segment (start 34.184846 23.89) (end 34.184846 23.27) (width 0.2) (layer "F.Cu") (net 7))
 (segment (start 34.424846 23.03) (end 34.544846 23.03) (width 0.2) (layer "F.Cu") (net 7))
 (segment (start 35.624846 23.03) (end 35.744846 23.03) (width 0.2) (layer "F.Cu") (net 7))
 (segment (start 36.811179 24.13) (end 41.86 24.13) (width 0.2) (layer "F.Cu") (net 7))
 (segment (start 35.024846 24.13) (end 35.144846 24.13) (width 0.2) (layer "F.Cu") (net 7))
 (segment (start 42.78 25.05) (end 44.105 25.05) (width 0.2) (layer "F.Cu") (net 7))
 (arc (start 34.784846 23.89) (mid 34.85514 24.059706) (end 35.024846 24.13) (width 0.2) (layer "F.Cu") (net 7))
 (arc (start 33.344846 23.03) (mid 33.514552 23.100294) (end 33.584846 23.27) (width 0.2) (layer "F.Cu") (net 7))
 (arc (start 35.144846 24.13) (mid 35.314552 24.059706) (end 35.384846 23.89) (width 0.2) (layer "F.Cu") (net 7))
 (arc (start 35.744846 23.03) (mid 35.914552 23.100294) (end 35.984846 23.27) (width 0.2) (layer "F.Cu") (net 7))
 (arc (start 35.384846 23.27) (mid 35.45514 23.100294) (end 35.624846 23.03) (width 0.2) (layer "F.Cu") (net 7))
 (arc (start 34.544846 23.03) (mid 34.714552 23.100294) (end 34.784846 23.27) (width 0.2) (layer "F.Cu") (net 7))
 (arc (start 33.944846 24.13) (mid 34.114552 24.059706) (end 34.184846 23.89) (width 0.2) (layer "F.Cu") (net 7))
 (arc (start 33.584846 23.89) (mid 33.65514 24.059706) (end 33.824846 24.13) (width 0.2) (layer "F.Cu") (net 7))
 (arc (start 32.984846 23.27) (mid 33.05514 23.100294) (end 33.224846 23.03) (width 0.2) (layer "F.Cu") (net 7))
 (arc (start 35.984846 23.89) (mid 36.05514 24.059706) (end 36.224846 24.13) (width 0.2) (layer "F.Cu") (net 7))
 (arc (start 32.744846 24.13) (mid 32.914552 24.059706) (end 32.984846 23.89) (width 0.2) (layer "F.Cu") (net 7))
 (arc (start 34.184846 23.27) (mid 34.25514 23.100294) (end 34.424846 23.03) (width 0.2) (layer "F.Cu") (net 7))
 (segment (start 29 24.07) (end 30.9675 24.07) (width 0.2) (layer "F.Cu") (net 2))
 (segment (start 30.9675 24.07) (end 33.5375 21.5) (width 0.2) (layer "F.Cu") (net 2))
 (segment (start 29 27.07) (end 31.7025 27.07) (width 0.2) (layer "F.Cu") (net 20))
 (segment (start 31.7025 27.07) (end 33.5375 25.235) (width 0.2) (layer "F.Cu") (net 20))
 (segment (start 42.24 25.59) (end 41.885 25.235) (width 0.2) (layer "F.Cu") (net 14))
 (segment (start 41.885 25.235) (end 40.5 25.235) (width 0.2) (layer "F.Cu") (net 14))
 (via (at 42.24 25.59) (size 0.6) (drill 0.3) (layers "F.Cu" "B.Cu") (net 14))
 (segment (start 42.24 25.59) (end 42.7 26.05) (width 0.2) (layer "B.Cu") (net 14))
 (segment (start 42.7 26.05) (end 44.105 26.05) (width 0.2) (layer "B.Cu") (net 14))
 (segment (start 40.5 22.2) (end 42.85 24.55) (width 0.2) (layer "F.Cu") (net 6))
 (segment (start 42.85 24.55) (end 44.105 24.55) (width 0.2) (layer "F.Cu") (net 6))
 (segment (start 40.5 21.5) (end 40.5 22.2) (width 0.2) (layer "F.Cu") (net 6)))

